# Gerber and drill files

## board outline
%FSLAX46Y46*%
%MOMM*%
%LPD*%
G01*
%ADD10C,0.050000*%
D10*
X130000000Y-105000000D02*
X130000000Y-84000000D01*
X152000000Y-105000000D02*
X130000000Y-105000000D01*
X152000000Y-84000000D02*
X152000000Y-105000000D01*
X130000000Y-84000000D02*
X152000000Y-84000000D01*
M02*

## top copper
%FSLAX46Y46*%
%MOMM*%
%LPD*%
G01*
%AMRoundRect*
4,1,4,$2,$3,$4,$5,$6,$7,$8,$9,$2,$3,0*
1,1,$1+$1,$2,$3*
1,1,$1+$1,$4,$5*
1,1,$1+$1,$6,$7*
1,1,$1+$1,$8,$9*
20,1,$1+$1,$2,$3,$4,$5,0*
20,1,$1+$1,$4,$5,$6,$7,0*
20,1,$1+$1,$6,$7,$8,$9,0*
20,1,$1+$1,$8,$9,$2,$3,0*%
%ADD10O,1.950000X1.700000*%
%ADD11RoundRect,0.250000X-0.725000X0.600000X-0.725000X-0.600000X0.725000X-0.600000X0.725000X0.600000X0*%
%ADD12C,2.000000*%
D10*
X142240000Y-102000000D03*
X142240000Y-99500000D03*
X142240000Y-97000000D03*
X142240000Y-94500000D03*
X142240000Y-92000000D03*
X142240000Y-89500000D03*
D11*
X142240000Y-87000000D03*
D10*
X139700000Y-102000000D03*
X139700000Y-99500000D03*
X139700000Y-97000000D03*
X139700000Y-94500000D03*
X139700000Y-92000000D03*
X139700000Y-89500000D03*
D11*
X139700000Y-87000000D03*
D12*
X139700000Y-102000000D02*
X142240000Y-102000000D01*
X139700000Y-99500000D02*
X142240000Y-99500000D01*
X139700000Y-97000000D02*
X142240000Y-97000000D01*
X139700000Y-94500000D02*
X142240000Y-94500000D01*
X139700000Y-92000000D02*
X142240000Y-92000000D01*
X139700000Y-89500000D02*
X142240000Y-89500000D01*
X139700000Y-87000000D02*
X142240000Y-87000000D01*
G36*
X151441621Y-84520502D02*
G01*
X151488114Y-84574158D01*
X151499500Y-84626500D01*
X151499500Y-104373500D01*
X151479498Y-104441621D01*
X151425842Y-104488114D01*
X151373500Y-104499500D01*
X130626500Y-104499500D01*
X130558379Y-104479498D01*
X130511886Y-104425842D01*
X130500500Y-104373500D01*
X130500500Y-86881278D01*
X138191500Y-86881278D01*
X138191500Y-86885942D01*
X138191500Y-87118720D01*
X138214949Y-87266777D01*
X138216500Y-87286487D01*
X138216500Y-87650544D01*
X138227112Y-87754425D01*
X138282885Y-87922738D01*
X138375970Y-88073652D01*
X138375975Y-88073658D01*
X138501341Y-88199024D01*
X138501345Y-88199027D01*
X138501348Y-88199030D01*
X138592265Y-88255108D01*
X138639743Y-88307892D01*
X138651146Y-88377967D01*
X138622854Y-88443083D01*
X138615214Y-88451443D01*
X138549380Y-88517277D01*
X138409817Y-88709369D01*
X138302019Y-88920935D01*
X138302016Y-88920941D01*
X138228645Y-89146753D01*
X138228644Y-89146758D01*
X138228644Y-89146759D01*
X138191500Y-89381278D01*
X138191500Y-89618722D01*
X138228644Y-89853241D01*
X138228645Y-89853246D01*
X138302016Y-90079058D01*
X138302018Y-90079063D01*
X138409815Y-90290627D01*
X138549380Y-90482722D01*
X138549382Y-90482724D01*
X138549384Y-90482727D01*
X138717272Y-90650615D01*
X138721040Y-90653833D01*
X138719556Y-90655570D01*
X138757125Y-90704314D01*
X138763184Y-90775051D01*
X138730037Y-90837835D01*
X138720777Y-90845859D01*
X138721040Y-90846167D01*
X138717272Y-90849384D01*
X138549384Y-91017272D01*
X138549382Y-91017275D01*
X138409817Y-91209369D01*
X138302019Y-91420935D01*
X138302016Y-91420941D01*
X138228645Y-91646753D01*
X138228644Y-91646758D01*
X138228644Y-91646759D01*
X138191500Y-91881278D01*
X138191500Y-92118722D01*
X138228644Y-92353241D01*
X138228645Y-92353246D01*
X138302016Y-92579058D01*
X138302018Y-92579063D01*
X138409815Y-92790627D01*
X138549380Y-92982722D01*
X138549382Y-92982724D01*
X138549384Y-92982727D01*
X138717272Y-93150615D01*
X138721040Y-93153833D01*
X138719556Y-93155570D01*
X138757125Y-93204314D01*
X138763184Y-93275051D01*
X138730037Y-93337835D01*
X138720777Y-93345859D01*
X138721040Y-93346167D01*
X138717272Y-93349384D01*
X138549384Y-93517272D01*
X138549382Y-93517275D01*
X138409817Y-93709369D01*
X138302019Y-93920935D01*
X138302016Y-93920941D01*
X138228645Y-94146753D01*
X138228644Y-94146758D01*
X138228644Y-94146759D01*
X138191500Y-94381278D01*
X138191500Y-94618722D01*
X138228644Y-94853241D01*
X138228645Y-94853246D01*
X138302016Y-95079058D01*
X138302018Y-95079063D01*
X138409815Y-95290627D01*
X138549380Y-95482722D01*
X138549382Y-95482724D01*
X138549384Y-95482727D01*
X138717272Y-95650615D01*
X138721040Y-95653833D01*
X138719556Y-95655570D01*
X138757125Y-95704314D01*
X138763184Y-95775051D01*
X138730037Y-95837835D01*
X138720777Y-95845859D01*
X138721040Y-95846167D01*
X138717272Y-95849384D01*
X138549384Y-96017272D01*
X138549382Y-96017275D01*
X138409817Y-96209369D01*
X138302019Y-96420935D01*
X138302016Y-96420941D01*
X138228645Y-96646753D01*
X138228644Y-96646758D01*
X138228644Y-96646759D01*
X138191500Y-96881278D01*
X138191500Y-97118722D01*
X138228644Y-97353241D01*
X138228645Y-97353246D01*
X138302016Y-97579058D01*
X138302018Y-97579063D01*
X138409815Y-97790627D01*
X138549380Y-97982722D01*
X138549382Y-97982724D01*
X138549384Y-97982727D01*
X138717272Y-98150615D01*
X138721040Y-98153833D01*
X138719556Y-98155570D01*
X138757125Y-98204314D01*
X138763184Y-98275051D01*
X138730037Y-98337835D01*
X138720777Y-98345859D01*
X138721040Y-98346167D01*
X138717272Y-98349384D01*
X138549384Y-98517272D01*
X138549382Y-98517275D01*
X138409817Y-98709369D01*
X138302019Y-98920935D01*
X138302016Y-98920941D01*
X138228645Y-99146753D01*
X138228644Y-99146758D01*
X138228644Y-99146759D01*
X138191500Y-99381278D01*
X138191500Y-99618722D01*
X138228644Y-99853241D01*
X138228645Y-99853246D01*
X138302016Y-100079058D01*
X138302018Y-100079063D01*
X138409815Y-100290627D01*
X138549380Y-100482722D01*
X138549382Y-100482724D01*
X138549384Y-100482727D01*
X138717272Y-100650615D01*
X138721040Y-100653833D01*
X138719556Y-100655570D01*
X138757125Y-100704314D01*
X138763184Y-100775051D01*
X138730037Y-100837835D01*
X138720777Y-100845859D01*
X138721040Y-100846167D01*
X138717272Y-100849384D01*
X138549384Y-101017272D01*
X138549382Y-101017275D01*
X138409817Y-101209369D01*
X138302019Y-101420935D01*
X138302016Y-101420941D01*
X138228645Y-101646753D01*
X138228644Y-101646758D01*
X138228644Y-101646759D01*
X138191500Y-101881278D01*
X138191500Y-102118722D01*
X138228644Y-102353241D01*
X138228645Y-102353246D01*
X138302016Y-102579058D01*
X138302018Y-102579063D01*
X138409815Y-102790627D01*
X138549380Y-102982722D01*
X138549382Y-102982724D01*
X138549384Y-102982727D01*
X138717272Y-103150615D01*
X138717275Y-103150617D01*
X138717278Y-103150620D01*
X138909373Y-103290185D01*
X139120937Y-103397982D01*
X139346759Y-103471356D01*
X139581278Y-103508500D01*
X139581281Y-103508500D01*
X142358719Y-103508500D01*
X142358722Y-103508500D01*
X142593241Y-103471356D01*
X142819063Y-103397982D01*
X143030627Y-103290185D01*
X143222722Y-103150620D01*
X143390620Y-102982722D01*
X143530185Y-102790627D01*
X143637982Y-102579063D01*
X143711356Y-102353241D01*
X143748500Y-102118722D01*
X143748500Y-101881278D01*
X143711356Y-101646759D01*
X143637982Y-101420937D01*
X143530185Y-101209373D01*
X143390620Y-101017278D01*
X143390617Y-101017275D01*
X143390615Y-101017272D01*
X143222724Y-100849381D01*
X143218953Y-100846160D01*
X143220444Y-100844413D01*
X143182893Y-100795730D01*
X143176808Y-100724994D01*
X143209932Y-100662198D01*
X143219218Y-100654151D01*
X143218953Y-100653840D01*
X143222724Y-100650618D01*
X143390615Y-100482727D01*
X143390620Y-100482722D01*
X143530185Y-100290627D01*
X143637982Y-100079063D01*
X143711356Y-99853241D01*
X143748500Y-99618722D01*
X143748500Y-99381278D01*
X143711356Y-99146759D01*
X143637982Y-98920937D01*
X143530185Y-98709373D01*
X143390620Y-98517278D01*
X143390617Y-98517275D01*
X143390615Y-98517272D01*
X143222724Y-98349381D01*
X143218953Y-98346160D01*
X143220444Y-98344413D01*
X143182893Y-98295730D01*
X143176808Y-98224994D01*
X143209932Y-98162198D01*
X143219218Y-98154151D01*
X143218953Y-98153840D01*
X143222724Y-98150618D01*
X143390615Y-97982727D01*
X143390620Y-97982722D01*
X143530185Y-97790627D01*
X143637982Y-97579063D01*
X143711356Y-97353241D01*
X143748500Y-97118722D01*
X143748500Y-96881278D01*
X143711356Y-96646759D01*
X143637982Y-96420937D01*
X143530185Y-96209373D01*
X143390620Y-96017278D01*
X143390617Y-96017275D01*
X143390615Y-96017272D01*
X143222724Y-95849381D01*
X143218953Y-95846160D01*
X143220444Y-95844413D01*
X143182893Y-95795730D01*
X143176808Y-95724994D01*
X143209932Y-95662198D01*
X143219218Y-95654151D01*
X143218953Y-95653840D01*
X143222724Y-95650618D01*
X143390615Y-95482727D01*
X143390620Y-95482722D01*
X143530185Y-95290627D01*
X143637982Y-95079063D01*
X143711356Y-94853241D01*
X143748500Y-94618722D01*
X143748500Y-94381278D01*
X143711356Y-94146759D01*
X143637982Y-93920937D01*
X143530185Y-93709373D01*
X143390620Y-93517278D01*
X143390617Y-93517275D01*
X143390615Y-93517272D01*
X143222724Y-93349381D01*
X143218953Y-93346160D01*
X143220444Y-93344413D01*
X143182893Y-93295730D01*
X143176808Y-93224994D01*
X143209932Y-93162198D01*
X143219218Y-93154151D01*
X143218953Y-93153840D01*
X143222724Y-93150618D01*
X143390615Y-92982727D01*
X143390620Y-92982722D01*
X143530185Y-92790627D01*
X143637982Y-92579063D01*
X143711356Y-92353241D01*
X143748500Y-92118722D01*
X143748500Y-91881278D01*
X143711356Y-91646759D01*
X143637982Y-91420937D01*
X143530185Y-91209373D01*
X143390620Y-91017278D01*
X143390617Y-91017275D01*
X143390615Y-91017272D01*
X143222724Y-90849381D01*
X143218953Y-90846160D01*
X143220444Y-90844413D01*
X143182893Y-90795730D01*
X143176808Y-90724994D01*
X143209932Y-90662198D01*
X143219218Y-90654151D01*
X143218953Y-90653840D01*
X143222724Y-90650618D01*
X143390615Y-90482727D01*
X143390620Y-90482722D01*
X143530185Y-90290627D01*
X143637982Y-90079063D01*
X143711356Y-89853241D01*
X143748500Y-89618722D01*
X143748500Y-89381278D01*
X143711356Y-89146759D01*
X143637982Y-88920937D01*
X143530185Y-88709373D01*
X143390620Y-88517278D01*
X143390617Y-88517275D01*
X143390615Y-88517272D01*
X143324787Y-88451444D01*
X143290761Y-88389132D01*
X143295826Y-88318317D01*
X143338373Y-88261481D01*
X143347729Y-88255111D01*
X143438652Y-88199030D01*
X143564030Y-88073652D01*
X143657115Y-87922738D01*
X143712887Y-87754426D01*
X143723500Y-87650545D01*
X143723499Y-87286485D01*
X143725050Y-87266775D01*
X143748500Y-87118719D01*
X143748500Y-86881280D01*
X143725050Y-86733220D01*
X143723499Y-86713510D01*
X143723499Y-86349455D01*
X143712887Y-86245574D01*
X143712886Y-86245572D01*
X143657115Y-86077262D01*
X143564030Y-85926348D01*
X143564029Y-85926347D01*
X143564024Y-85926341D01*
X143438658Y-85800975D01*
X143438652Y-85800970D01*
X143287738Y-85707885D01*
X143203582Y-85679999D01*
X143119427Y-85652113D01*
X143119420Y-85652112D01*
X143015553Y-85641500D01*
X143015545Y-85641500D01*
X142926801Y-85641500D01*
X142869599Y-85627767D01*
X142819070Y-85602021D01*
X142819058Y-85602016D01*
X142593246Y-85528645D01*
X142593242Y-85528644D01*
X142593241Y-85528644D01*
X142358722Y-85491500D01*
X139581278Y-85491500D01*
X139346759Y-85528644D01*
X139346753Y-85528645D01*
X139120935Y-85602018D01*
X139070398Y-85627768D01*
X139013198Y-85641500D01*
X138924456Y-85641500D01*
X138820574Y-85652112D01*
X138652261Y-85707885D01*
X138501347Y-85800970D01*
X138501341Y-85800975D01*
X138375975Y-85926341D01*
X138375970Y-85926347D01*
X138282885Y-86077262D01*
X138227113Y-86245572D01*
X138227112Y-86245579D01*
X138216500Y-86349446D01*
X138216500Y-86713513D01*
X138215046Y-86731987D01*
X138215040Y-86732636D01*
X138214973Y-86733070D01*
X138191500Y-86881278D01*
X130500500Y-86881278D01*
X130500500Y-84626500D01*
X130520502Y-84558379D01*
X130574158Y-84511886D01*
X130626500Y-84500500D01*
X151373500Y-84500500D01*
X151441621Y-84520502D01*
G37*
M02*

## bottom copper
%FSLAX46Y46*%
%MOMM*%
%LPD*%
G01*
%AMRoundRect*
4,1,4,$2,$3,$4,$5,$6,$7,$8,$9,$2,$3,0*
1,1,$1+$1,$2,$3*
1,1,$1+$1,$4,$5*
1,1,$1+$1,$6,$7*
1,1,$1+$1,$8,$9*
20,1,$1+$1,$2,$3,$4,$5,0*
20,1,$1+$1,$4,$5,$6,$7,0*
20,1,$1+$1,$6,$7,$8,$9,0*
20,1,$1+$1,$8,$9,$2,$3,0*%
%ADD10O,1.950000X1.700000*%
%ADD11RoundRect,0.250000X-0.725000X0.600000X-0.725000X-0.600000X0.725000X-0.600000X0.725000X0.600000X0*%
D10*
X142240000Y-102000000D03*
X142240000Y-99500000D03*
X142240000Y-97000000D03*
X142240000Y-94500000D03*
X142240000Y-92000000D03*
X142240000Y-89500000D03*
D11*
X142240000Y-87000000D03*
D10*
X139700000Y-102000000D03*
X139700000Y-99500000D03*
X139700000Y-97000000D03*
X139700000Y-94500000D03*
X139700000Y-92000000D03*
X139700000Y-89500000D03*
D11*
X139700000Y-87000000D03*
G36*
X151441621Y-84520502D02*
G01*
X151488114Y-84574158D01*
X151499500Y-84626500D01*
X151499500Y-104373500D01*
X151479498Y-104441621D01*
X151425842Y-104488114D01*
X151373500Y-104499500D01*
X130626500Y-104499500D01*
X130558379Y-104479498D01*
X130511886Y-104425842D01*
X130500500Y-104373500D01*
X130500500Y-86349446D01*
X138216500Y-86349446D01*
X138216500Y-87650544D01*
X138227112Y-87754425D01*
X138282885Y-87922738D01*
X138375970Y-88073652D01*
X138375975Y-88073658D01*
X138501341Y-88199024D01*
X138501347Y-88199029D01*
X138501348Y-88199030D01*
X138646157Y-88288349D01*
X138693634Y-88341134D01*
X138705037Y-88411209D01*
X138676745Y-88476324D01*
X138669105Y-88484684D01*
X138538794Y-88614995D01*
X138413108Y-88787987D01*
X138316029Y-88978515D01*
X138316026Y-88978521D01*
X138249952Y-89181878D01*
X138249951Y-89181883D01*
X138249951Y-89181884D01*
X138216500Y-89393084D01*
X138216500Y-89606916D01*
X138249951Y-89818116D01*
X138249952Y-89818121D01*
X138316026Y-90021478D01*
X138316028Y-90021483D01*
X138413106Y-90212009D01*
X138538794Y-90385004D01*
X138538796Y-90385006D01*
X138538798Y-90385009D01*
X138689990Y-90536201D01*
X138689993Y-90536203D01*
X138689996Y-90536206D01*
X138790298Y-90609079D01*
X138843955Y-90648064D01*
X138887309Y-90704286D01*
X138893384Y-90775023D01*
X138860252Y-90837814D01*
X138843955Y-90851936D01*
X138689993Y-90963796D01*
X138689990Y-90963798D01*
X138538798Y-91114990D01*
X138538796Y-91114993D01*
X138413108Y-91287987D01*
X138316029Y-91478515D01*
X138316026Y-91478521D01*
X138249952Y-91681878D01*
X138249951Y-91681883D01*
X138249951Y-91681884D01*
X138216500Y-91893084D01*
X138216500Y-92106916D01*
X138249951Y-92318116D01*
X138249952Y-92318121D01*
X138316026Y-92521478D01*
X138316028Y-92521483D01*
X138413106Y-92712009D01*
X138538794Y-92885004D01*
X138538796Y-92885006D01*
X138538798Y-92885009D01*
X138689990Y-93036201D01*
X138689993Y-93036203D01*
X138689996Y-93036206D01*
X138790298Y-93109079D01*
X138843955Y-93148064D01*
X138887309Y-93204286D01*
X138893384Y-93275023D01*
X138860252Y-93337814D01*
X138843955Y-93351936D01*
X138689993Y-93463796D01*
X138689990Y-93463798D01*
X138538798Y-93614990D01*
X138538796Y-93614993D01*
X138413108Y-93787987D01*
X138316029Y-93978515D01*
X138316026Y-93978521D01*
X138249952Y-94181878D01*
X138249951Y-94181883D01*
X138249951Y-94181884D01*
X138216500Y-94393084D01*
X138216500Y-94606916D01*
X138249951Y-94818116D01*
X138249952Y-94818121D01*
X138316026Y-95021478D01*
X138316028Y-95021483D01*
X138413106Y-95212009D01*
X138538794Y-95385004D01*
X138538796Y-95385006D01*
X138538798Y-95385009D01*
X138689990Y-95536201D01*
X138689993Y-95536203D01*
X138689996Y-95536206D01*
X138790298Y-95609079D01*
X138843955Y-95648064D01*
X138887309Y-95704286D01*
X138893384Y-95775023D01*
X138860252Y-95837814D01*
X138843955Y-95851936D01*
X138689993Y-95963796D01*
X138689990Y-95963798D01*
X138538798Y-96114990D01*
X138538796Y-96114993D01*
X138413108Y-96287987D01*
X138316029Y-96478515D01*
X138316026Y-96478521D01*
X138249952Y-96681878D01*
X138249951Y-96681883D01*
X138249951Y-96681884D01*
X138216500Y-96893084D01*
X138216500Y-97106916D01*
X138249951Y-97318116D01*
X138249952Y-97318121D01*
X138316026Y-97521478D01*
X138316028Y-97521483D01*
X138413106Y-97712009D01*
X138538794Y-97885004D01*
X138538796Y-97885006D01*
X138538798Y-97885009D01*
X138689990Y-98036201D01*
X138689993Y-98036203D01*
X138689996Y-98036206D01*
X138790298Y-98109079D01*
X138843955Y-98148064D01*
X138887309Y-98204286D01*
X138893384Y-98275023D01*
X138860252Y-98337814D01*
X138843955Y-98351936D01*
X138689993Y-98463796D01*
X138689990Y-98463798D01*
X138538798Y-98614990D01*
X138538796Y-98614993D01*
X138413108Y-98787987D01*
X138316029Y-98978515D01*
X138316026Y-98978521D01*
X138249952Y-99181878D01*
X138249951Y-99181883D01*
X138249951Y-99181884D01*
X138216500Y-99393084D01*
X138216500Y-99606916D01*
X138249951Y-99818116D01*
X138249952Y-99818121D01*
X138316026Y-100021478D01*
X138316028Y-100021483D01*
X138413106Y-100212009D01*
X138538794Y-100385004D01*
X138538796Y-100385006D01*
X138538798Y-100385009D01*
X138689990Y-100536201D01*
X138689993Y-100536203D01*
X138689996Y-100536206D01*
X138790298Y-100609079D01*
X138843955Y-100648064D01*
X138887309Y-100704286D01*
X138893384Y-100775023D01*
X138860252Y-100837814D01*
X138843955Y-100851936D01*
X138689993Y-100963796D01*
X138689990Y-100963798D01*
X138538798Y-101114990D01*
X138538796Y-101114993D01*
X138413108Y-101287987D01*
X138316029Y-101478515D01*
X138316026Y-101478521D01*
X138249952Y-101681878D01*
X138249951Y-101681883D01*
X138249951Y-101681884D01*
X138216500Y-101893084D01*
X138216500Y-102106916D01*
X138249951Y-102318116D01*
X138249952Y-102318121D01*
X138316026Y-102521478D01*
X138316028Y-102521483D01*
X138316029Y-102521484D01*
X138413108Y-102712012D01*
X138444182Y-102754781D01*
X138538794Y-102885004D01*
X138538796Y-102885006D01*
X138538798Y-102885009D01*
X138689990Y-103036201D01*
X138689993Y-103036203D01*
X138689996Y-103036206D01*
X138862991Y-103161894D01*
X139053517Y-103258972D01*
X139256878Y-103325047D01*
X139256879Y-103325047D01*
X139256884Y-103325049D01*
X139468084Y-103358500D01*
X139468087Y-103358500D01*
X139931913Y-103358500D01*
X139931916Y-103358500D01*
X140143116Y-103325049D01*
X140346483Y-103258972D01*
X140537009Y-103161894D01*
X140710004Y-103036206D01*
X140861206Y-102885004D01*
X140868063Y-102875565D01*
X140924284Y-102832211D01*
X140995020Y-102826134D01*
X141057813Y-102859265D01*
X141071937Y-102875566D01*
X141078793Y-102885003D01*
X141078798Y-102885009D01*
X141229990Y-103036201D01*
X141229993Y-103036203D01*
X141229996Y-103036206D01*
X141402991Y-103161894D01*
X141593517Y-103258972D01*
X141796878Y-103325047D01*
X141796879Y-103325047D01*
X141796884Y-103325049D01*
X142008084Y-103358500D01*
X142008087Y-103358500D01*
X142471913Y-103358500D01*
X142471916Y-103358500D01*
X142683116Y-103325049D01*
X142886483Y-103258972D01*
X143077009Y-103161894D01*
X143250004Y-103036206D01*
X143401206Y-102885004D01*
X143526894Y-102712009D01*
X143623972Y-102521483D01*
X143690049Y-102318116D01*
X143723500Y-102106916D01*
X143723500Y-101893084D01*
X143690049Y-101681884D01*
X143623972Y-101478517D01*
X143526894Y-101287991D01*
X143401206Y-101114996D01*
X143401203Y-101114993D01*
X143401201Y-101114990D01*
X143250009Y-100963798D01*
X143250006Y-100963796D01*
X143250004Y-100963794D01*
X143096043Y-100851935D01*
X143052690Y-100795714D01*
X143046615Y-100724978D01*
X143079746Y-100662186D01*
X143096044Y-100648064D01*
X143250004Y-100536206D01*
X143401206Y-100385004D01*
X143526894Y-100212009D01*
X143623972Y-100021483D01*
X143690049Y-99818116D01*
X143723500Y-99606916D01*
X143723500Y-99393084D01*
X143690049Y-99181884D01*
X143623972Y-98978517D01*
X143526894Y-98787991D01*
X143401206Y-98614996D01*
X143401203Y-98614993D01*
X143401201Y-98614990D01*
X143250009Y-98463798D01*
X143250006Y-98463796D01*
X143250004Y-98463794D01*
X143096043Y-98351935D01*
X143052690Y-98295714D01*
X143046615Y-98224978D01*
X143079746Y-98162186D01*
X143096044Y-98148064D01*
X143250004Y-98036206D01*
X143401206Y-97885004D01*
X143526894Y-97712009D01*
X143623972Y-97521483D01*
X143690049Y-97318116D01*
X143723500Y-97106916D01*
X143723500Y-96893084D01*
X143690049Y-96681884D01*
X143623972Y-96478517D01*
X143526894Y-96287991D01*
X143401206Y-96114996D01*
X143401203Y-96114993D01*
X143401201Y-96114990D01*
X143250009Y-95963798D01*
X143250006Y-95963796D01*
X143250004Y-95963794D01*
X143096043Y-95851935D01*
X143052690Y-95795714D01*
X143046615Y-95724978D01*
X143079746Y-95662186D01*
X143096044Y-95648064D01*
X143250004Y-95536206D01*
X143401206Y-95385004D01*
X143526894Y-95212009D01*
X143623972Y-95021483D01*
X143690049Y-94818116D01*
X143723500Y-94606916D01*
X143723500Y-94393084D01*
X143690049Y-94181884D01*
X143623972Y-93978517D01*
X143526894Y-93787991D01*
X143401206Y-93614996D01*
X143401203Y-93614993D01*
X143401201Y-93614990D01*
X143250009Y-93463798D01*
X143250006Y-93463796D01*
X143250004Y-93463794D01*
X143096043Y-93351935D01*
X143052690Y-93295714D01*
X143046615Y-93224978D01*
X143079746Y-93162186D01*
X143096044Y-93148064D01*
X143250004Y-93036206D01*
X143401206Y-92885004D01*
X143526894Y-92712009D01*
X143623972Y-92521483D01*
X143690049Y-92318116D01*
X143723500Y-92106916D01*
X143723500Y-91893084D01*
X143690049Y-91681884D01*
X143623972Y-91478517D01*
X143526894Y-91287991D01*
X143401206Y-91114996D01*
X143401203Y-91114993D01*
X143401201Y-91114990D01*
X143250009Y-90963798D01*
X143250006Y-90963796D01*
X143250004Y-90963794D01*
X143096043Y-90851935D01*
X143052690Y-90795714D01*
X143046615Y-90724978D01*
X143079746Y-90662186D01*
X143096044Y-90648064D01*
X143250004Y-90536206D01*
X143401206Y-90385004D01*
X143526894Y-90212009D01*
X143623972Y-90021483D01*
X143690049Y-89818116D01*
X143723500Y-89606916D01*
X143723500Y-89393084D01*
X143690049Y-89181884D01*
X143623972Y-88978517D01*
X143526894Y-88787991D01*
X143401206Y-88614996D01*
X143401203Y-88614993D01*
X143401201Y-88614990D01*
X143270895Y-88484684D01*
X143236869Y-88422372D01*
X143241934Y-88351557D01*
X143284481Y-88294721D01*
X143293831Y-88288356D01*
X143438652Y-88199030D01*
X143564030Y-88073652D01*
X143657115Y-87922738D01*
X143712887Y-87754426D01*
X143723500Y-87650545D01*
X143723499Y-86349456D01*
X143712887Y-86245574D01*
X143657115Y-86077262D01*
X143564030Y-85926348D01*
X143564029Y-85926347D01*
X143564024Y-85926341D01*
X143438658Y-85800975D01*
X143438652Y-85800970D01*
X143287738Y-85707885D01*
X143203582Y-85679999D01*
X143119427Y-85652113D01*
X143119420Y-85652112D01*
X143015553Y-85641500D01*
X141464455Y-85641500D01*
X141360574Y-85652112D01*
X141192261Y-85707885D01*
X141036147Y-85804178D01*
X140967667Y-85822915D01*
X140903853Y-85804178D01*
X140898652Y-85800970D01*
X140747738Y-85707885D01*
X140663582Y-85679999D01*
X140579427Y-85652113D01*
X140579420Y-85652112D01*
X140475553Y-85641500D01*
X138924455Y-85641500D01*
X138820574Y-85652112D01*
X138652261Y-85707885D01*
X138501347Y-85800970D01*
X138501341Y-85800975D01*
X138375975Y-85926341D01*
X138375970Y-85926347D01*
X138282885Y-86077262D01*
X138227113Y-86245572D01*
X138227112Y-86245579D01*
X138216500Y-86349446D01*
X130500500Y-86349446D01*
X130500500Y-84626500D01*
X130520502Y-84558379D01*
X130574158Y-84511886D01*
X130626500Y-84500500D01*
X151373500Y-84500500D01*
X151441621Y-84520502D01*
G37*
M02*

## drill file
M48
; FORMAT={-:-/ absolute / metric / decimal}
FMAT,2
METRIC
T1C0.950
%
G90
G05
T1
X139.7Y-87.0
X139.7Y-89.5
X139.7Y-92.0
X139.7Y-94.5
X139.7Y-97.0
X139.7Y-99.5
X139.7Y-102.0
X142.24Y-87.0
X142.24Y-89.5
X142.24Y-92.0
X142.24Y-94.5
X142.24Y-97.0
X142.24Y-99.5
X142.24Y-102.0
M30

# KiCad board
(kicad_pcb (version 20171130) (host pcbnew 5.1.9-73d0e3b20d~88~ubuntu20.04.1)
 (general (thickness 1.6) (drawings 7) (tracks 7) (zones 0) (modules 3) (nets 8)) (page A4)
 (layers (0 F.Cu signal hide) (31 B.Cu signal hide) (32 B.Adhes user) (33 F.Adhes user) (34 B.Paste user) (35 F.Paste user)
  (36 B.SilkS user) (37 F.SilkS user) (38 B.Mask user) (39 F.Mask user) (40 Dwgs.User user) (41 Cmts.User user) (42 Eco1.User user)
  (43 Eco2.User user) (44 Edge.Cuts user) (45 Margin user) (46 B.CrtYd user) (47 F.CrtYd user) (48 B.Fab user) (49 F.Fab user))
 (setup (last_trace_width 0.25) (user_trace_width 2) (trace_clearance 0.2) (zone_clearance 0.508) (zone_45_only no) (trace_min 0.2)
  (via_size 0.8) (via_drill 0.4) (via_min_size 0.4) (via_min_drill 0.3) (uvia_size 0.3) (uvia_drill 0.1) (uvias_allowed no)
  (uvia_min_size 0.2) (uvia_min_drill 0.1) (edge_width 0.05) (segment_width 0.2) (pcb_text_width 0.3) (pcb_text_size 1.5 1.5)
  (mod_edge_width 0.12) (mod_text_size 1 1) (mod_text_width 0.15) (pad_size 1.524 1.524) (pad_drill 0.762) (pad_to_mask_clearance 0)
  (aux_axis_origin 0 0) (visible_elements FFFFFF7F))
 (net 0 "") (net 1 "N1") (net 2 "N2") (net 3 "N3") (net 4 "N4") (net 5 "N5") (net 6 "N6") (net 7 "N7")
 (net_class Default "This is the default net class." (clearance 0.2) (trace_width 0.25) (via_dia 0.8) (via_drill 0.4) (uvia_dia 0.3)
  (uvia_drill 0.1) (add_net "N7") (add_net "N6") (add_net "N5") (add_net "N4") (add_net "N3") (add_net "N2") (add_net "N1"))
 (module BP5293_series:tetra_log (layer F.Cu) (at 146 94.7 90)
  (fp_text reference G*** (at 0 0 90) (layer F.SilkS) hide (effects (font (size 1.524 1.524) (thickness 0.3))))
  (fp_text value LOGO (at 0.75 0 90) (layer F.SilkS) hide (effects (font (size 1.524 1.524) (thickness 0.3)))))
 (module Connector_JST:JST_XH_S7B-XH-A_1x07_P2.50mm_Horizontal (layer B.Cu) (at 142.24 87 270)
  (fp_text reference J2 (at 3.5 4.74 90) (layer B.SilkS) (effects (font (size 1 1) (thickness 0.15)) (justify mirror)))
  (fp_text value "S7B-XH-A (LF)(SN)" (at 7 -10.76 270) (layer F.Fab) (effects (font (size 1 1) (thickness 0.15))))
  (pad 7 thru_hole oval (at 15 0 270) (size 1.7 1.95) (drill 0.95) (layers *.Cu *.Mask) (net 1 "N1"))
  (pad 6 thru_hole oval (at 12.5 0 270) (size 1.7 1.95) (drill 0.95) (layers *.Cu *.Mask) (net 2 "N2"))
  (pad 5 thru_hole oval (at 10 0 270) (size 1.7 1.95) (drill 0.95) (layers *.Cu *.Mask) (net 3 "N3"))
  (pad 4 thru_hole oval (at 7.5 0 270) (size 1.7 1.95) (drill 0.95) (layers *.Cu *.Mask) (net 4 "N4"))
  (pad 3 thru_hole oval (at 5 0 270) (size 1.7 1.95) (drill 0.95) (layers *.Cu *.Mask) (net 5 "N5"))
  (pad 2 thru_hole oval (at 2.5 0 270) (size 1.7 1.95) (drill 0.95) (layers *.Cu *.Mask) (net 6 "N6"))
  (pad 1 thru_hole roundrect (at 0 0 270) (size 1.7 1.95) (drill 0.95) (layers *.Cu *.Mask) (roundrect_rratio 0.1470588235294118)
   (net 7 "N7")))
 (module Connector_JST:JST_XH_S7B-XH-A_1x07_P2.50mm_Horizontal (layer F.Cu) (at 139.7 87 270)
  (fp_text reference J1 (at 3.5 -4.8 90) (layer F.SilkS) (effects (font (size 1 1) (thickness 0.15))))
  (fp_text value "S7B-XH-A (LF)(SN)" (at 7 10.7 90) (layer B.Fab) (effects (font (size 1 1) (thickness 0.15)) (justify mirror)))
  (pad 7 thru_hole oval (at 15 0 270) (size 1.7 1.95) (drill 0.95) (layers *.Cu *.Mask) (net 1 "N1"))
  (pad 6 thru_hole oval (at 12.5 0 270) (size 1.7 1.95) (drill 0.95) (layers *.Cu *.Mask) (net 2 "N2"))
  (pad 5 thru_hole oval (at 10 0 270) (size 1.7 1.95) (drill 0.95) (layers *.Cu *.Mask) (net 3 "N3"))
  (pad 4 thru_hole oval (at 7.5 0 270) (size 1.7 1.95) (drill 0.95) (layers *.Cu *.Mask) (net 4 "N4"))
  (pad 3 thru_hole oval (at 5 0 270) (size 1.7 1.95) (drill 0.95) (layers *.Cu *.Mask) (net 5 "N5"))
  (pad 2 thru_hole oval (at 2.5 0 270) (size 1.7 1.95) (drill 0.95) (layers *.Cu *.Mask) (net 6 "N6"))
  (pad 1 thru_hole roundrect (at 0 0 270) (size 1.7 1.95) (drill 0.95) (layers *.Cu *.Mask) (roundrect_rratio 0.1470588235294118)
   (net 7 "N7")))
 (gr_line (start 130 105) (end 130 84) (layer Edge.Cuts) (width 0.05))
 (gr_line (start 152 105) (end 130 105) (layer Edge.Cuts) (width 0.05))
 (gr_line (start 152 84) (end 152 105) (layer Edge.Cuts) (width 0.05))
 (gr_line (start 130 84) (end 152 84) (layer Edge.Cuts) (width 0.05))
 (segment (start 139.7 102) (end 142.24 102) (width 2) (layer F.Cu) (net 1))
 (segment (start 139.7 99.5) (end 142.24 99.5) (width 2) (layer F.Cu) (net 2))
 (segment (start 139.7 97) (end 142.24 97) (width 2) (layer F.Cu) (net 3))
 (segment (start 139.7 94.5) (end 142.24 94.5) (width 2) (layer F.Cu) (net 4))
 (segment (start 139.7 92) (end 142.24 92) (width 2) (layer F.Cu) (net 5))
 (segment (start 139.7 89.5) (end 142.24 89.5) (width 2) (layer F.Cu) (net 6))
 (segment (start 139.7 87) (end 142.24 87) (width 2) (layer F.Cu) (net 7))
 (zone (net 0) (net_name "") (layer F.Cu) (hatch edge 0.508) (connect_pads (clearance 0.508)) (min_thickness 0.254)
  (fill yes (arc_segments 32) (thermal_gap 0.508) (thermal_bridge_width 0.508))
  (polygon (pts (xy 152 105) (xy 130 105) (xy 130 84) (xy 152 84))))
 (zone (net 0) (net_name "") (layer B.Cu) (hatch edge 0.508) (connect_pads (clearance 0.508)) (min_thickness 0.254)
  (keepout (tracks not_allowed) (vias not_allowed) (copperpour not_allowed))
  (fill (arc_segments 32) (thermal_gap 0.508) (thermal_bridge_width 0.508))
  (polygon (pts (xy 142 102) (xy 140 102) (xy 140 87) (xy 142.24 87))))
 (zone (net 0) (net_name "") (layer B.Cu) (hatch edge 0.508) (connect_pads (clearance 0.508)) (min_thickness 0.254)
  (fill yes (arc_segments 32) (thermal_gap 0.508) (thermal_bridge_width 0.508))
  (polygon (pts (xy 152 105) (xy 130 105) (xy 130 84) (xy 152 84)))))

